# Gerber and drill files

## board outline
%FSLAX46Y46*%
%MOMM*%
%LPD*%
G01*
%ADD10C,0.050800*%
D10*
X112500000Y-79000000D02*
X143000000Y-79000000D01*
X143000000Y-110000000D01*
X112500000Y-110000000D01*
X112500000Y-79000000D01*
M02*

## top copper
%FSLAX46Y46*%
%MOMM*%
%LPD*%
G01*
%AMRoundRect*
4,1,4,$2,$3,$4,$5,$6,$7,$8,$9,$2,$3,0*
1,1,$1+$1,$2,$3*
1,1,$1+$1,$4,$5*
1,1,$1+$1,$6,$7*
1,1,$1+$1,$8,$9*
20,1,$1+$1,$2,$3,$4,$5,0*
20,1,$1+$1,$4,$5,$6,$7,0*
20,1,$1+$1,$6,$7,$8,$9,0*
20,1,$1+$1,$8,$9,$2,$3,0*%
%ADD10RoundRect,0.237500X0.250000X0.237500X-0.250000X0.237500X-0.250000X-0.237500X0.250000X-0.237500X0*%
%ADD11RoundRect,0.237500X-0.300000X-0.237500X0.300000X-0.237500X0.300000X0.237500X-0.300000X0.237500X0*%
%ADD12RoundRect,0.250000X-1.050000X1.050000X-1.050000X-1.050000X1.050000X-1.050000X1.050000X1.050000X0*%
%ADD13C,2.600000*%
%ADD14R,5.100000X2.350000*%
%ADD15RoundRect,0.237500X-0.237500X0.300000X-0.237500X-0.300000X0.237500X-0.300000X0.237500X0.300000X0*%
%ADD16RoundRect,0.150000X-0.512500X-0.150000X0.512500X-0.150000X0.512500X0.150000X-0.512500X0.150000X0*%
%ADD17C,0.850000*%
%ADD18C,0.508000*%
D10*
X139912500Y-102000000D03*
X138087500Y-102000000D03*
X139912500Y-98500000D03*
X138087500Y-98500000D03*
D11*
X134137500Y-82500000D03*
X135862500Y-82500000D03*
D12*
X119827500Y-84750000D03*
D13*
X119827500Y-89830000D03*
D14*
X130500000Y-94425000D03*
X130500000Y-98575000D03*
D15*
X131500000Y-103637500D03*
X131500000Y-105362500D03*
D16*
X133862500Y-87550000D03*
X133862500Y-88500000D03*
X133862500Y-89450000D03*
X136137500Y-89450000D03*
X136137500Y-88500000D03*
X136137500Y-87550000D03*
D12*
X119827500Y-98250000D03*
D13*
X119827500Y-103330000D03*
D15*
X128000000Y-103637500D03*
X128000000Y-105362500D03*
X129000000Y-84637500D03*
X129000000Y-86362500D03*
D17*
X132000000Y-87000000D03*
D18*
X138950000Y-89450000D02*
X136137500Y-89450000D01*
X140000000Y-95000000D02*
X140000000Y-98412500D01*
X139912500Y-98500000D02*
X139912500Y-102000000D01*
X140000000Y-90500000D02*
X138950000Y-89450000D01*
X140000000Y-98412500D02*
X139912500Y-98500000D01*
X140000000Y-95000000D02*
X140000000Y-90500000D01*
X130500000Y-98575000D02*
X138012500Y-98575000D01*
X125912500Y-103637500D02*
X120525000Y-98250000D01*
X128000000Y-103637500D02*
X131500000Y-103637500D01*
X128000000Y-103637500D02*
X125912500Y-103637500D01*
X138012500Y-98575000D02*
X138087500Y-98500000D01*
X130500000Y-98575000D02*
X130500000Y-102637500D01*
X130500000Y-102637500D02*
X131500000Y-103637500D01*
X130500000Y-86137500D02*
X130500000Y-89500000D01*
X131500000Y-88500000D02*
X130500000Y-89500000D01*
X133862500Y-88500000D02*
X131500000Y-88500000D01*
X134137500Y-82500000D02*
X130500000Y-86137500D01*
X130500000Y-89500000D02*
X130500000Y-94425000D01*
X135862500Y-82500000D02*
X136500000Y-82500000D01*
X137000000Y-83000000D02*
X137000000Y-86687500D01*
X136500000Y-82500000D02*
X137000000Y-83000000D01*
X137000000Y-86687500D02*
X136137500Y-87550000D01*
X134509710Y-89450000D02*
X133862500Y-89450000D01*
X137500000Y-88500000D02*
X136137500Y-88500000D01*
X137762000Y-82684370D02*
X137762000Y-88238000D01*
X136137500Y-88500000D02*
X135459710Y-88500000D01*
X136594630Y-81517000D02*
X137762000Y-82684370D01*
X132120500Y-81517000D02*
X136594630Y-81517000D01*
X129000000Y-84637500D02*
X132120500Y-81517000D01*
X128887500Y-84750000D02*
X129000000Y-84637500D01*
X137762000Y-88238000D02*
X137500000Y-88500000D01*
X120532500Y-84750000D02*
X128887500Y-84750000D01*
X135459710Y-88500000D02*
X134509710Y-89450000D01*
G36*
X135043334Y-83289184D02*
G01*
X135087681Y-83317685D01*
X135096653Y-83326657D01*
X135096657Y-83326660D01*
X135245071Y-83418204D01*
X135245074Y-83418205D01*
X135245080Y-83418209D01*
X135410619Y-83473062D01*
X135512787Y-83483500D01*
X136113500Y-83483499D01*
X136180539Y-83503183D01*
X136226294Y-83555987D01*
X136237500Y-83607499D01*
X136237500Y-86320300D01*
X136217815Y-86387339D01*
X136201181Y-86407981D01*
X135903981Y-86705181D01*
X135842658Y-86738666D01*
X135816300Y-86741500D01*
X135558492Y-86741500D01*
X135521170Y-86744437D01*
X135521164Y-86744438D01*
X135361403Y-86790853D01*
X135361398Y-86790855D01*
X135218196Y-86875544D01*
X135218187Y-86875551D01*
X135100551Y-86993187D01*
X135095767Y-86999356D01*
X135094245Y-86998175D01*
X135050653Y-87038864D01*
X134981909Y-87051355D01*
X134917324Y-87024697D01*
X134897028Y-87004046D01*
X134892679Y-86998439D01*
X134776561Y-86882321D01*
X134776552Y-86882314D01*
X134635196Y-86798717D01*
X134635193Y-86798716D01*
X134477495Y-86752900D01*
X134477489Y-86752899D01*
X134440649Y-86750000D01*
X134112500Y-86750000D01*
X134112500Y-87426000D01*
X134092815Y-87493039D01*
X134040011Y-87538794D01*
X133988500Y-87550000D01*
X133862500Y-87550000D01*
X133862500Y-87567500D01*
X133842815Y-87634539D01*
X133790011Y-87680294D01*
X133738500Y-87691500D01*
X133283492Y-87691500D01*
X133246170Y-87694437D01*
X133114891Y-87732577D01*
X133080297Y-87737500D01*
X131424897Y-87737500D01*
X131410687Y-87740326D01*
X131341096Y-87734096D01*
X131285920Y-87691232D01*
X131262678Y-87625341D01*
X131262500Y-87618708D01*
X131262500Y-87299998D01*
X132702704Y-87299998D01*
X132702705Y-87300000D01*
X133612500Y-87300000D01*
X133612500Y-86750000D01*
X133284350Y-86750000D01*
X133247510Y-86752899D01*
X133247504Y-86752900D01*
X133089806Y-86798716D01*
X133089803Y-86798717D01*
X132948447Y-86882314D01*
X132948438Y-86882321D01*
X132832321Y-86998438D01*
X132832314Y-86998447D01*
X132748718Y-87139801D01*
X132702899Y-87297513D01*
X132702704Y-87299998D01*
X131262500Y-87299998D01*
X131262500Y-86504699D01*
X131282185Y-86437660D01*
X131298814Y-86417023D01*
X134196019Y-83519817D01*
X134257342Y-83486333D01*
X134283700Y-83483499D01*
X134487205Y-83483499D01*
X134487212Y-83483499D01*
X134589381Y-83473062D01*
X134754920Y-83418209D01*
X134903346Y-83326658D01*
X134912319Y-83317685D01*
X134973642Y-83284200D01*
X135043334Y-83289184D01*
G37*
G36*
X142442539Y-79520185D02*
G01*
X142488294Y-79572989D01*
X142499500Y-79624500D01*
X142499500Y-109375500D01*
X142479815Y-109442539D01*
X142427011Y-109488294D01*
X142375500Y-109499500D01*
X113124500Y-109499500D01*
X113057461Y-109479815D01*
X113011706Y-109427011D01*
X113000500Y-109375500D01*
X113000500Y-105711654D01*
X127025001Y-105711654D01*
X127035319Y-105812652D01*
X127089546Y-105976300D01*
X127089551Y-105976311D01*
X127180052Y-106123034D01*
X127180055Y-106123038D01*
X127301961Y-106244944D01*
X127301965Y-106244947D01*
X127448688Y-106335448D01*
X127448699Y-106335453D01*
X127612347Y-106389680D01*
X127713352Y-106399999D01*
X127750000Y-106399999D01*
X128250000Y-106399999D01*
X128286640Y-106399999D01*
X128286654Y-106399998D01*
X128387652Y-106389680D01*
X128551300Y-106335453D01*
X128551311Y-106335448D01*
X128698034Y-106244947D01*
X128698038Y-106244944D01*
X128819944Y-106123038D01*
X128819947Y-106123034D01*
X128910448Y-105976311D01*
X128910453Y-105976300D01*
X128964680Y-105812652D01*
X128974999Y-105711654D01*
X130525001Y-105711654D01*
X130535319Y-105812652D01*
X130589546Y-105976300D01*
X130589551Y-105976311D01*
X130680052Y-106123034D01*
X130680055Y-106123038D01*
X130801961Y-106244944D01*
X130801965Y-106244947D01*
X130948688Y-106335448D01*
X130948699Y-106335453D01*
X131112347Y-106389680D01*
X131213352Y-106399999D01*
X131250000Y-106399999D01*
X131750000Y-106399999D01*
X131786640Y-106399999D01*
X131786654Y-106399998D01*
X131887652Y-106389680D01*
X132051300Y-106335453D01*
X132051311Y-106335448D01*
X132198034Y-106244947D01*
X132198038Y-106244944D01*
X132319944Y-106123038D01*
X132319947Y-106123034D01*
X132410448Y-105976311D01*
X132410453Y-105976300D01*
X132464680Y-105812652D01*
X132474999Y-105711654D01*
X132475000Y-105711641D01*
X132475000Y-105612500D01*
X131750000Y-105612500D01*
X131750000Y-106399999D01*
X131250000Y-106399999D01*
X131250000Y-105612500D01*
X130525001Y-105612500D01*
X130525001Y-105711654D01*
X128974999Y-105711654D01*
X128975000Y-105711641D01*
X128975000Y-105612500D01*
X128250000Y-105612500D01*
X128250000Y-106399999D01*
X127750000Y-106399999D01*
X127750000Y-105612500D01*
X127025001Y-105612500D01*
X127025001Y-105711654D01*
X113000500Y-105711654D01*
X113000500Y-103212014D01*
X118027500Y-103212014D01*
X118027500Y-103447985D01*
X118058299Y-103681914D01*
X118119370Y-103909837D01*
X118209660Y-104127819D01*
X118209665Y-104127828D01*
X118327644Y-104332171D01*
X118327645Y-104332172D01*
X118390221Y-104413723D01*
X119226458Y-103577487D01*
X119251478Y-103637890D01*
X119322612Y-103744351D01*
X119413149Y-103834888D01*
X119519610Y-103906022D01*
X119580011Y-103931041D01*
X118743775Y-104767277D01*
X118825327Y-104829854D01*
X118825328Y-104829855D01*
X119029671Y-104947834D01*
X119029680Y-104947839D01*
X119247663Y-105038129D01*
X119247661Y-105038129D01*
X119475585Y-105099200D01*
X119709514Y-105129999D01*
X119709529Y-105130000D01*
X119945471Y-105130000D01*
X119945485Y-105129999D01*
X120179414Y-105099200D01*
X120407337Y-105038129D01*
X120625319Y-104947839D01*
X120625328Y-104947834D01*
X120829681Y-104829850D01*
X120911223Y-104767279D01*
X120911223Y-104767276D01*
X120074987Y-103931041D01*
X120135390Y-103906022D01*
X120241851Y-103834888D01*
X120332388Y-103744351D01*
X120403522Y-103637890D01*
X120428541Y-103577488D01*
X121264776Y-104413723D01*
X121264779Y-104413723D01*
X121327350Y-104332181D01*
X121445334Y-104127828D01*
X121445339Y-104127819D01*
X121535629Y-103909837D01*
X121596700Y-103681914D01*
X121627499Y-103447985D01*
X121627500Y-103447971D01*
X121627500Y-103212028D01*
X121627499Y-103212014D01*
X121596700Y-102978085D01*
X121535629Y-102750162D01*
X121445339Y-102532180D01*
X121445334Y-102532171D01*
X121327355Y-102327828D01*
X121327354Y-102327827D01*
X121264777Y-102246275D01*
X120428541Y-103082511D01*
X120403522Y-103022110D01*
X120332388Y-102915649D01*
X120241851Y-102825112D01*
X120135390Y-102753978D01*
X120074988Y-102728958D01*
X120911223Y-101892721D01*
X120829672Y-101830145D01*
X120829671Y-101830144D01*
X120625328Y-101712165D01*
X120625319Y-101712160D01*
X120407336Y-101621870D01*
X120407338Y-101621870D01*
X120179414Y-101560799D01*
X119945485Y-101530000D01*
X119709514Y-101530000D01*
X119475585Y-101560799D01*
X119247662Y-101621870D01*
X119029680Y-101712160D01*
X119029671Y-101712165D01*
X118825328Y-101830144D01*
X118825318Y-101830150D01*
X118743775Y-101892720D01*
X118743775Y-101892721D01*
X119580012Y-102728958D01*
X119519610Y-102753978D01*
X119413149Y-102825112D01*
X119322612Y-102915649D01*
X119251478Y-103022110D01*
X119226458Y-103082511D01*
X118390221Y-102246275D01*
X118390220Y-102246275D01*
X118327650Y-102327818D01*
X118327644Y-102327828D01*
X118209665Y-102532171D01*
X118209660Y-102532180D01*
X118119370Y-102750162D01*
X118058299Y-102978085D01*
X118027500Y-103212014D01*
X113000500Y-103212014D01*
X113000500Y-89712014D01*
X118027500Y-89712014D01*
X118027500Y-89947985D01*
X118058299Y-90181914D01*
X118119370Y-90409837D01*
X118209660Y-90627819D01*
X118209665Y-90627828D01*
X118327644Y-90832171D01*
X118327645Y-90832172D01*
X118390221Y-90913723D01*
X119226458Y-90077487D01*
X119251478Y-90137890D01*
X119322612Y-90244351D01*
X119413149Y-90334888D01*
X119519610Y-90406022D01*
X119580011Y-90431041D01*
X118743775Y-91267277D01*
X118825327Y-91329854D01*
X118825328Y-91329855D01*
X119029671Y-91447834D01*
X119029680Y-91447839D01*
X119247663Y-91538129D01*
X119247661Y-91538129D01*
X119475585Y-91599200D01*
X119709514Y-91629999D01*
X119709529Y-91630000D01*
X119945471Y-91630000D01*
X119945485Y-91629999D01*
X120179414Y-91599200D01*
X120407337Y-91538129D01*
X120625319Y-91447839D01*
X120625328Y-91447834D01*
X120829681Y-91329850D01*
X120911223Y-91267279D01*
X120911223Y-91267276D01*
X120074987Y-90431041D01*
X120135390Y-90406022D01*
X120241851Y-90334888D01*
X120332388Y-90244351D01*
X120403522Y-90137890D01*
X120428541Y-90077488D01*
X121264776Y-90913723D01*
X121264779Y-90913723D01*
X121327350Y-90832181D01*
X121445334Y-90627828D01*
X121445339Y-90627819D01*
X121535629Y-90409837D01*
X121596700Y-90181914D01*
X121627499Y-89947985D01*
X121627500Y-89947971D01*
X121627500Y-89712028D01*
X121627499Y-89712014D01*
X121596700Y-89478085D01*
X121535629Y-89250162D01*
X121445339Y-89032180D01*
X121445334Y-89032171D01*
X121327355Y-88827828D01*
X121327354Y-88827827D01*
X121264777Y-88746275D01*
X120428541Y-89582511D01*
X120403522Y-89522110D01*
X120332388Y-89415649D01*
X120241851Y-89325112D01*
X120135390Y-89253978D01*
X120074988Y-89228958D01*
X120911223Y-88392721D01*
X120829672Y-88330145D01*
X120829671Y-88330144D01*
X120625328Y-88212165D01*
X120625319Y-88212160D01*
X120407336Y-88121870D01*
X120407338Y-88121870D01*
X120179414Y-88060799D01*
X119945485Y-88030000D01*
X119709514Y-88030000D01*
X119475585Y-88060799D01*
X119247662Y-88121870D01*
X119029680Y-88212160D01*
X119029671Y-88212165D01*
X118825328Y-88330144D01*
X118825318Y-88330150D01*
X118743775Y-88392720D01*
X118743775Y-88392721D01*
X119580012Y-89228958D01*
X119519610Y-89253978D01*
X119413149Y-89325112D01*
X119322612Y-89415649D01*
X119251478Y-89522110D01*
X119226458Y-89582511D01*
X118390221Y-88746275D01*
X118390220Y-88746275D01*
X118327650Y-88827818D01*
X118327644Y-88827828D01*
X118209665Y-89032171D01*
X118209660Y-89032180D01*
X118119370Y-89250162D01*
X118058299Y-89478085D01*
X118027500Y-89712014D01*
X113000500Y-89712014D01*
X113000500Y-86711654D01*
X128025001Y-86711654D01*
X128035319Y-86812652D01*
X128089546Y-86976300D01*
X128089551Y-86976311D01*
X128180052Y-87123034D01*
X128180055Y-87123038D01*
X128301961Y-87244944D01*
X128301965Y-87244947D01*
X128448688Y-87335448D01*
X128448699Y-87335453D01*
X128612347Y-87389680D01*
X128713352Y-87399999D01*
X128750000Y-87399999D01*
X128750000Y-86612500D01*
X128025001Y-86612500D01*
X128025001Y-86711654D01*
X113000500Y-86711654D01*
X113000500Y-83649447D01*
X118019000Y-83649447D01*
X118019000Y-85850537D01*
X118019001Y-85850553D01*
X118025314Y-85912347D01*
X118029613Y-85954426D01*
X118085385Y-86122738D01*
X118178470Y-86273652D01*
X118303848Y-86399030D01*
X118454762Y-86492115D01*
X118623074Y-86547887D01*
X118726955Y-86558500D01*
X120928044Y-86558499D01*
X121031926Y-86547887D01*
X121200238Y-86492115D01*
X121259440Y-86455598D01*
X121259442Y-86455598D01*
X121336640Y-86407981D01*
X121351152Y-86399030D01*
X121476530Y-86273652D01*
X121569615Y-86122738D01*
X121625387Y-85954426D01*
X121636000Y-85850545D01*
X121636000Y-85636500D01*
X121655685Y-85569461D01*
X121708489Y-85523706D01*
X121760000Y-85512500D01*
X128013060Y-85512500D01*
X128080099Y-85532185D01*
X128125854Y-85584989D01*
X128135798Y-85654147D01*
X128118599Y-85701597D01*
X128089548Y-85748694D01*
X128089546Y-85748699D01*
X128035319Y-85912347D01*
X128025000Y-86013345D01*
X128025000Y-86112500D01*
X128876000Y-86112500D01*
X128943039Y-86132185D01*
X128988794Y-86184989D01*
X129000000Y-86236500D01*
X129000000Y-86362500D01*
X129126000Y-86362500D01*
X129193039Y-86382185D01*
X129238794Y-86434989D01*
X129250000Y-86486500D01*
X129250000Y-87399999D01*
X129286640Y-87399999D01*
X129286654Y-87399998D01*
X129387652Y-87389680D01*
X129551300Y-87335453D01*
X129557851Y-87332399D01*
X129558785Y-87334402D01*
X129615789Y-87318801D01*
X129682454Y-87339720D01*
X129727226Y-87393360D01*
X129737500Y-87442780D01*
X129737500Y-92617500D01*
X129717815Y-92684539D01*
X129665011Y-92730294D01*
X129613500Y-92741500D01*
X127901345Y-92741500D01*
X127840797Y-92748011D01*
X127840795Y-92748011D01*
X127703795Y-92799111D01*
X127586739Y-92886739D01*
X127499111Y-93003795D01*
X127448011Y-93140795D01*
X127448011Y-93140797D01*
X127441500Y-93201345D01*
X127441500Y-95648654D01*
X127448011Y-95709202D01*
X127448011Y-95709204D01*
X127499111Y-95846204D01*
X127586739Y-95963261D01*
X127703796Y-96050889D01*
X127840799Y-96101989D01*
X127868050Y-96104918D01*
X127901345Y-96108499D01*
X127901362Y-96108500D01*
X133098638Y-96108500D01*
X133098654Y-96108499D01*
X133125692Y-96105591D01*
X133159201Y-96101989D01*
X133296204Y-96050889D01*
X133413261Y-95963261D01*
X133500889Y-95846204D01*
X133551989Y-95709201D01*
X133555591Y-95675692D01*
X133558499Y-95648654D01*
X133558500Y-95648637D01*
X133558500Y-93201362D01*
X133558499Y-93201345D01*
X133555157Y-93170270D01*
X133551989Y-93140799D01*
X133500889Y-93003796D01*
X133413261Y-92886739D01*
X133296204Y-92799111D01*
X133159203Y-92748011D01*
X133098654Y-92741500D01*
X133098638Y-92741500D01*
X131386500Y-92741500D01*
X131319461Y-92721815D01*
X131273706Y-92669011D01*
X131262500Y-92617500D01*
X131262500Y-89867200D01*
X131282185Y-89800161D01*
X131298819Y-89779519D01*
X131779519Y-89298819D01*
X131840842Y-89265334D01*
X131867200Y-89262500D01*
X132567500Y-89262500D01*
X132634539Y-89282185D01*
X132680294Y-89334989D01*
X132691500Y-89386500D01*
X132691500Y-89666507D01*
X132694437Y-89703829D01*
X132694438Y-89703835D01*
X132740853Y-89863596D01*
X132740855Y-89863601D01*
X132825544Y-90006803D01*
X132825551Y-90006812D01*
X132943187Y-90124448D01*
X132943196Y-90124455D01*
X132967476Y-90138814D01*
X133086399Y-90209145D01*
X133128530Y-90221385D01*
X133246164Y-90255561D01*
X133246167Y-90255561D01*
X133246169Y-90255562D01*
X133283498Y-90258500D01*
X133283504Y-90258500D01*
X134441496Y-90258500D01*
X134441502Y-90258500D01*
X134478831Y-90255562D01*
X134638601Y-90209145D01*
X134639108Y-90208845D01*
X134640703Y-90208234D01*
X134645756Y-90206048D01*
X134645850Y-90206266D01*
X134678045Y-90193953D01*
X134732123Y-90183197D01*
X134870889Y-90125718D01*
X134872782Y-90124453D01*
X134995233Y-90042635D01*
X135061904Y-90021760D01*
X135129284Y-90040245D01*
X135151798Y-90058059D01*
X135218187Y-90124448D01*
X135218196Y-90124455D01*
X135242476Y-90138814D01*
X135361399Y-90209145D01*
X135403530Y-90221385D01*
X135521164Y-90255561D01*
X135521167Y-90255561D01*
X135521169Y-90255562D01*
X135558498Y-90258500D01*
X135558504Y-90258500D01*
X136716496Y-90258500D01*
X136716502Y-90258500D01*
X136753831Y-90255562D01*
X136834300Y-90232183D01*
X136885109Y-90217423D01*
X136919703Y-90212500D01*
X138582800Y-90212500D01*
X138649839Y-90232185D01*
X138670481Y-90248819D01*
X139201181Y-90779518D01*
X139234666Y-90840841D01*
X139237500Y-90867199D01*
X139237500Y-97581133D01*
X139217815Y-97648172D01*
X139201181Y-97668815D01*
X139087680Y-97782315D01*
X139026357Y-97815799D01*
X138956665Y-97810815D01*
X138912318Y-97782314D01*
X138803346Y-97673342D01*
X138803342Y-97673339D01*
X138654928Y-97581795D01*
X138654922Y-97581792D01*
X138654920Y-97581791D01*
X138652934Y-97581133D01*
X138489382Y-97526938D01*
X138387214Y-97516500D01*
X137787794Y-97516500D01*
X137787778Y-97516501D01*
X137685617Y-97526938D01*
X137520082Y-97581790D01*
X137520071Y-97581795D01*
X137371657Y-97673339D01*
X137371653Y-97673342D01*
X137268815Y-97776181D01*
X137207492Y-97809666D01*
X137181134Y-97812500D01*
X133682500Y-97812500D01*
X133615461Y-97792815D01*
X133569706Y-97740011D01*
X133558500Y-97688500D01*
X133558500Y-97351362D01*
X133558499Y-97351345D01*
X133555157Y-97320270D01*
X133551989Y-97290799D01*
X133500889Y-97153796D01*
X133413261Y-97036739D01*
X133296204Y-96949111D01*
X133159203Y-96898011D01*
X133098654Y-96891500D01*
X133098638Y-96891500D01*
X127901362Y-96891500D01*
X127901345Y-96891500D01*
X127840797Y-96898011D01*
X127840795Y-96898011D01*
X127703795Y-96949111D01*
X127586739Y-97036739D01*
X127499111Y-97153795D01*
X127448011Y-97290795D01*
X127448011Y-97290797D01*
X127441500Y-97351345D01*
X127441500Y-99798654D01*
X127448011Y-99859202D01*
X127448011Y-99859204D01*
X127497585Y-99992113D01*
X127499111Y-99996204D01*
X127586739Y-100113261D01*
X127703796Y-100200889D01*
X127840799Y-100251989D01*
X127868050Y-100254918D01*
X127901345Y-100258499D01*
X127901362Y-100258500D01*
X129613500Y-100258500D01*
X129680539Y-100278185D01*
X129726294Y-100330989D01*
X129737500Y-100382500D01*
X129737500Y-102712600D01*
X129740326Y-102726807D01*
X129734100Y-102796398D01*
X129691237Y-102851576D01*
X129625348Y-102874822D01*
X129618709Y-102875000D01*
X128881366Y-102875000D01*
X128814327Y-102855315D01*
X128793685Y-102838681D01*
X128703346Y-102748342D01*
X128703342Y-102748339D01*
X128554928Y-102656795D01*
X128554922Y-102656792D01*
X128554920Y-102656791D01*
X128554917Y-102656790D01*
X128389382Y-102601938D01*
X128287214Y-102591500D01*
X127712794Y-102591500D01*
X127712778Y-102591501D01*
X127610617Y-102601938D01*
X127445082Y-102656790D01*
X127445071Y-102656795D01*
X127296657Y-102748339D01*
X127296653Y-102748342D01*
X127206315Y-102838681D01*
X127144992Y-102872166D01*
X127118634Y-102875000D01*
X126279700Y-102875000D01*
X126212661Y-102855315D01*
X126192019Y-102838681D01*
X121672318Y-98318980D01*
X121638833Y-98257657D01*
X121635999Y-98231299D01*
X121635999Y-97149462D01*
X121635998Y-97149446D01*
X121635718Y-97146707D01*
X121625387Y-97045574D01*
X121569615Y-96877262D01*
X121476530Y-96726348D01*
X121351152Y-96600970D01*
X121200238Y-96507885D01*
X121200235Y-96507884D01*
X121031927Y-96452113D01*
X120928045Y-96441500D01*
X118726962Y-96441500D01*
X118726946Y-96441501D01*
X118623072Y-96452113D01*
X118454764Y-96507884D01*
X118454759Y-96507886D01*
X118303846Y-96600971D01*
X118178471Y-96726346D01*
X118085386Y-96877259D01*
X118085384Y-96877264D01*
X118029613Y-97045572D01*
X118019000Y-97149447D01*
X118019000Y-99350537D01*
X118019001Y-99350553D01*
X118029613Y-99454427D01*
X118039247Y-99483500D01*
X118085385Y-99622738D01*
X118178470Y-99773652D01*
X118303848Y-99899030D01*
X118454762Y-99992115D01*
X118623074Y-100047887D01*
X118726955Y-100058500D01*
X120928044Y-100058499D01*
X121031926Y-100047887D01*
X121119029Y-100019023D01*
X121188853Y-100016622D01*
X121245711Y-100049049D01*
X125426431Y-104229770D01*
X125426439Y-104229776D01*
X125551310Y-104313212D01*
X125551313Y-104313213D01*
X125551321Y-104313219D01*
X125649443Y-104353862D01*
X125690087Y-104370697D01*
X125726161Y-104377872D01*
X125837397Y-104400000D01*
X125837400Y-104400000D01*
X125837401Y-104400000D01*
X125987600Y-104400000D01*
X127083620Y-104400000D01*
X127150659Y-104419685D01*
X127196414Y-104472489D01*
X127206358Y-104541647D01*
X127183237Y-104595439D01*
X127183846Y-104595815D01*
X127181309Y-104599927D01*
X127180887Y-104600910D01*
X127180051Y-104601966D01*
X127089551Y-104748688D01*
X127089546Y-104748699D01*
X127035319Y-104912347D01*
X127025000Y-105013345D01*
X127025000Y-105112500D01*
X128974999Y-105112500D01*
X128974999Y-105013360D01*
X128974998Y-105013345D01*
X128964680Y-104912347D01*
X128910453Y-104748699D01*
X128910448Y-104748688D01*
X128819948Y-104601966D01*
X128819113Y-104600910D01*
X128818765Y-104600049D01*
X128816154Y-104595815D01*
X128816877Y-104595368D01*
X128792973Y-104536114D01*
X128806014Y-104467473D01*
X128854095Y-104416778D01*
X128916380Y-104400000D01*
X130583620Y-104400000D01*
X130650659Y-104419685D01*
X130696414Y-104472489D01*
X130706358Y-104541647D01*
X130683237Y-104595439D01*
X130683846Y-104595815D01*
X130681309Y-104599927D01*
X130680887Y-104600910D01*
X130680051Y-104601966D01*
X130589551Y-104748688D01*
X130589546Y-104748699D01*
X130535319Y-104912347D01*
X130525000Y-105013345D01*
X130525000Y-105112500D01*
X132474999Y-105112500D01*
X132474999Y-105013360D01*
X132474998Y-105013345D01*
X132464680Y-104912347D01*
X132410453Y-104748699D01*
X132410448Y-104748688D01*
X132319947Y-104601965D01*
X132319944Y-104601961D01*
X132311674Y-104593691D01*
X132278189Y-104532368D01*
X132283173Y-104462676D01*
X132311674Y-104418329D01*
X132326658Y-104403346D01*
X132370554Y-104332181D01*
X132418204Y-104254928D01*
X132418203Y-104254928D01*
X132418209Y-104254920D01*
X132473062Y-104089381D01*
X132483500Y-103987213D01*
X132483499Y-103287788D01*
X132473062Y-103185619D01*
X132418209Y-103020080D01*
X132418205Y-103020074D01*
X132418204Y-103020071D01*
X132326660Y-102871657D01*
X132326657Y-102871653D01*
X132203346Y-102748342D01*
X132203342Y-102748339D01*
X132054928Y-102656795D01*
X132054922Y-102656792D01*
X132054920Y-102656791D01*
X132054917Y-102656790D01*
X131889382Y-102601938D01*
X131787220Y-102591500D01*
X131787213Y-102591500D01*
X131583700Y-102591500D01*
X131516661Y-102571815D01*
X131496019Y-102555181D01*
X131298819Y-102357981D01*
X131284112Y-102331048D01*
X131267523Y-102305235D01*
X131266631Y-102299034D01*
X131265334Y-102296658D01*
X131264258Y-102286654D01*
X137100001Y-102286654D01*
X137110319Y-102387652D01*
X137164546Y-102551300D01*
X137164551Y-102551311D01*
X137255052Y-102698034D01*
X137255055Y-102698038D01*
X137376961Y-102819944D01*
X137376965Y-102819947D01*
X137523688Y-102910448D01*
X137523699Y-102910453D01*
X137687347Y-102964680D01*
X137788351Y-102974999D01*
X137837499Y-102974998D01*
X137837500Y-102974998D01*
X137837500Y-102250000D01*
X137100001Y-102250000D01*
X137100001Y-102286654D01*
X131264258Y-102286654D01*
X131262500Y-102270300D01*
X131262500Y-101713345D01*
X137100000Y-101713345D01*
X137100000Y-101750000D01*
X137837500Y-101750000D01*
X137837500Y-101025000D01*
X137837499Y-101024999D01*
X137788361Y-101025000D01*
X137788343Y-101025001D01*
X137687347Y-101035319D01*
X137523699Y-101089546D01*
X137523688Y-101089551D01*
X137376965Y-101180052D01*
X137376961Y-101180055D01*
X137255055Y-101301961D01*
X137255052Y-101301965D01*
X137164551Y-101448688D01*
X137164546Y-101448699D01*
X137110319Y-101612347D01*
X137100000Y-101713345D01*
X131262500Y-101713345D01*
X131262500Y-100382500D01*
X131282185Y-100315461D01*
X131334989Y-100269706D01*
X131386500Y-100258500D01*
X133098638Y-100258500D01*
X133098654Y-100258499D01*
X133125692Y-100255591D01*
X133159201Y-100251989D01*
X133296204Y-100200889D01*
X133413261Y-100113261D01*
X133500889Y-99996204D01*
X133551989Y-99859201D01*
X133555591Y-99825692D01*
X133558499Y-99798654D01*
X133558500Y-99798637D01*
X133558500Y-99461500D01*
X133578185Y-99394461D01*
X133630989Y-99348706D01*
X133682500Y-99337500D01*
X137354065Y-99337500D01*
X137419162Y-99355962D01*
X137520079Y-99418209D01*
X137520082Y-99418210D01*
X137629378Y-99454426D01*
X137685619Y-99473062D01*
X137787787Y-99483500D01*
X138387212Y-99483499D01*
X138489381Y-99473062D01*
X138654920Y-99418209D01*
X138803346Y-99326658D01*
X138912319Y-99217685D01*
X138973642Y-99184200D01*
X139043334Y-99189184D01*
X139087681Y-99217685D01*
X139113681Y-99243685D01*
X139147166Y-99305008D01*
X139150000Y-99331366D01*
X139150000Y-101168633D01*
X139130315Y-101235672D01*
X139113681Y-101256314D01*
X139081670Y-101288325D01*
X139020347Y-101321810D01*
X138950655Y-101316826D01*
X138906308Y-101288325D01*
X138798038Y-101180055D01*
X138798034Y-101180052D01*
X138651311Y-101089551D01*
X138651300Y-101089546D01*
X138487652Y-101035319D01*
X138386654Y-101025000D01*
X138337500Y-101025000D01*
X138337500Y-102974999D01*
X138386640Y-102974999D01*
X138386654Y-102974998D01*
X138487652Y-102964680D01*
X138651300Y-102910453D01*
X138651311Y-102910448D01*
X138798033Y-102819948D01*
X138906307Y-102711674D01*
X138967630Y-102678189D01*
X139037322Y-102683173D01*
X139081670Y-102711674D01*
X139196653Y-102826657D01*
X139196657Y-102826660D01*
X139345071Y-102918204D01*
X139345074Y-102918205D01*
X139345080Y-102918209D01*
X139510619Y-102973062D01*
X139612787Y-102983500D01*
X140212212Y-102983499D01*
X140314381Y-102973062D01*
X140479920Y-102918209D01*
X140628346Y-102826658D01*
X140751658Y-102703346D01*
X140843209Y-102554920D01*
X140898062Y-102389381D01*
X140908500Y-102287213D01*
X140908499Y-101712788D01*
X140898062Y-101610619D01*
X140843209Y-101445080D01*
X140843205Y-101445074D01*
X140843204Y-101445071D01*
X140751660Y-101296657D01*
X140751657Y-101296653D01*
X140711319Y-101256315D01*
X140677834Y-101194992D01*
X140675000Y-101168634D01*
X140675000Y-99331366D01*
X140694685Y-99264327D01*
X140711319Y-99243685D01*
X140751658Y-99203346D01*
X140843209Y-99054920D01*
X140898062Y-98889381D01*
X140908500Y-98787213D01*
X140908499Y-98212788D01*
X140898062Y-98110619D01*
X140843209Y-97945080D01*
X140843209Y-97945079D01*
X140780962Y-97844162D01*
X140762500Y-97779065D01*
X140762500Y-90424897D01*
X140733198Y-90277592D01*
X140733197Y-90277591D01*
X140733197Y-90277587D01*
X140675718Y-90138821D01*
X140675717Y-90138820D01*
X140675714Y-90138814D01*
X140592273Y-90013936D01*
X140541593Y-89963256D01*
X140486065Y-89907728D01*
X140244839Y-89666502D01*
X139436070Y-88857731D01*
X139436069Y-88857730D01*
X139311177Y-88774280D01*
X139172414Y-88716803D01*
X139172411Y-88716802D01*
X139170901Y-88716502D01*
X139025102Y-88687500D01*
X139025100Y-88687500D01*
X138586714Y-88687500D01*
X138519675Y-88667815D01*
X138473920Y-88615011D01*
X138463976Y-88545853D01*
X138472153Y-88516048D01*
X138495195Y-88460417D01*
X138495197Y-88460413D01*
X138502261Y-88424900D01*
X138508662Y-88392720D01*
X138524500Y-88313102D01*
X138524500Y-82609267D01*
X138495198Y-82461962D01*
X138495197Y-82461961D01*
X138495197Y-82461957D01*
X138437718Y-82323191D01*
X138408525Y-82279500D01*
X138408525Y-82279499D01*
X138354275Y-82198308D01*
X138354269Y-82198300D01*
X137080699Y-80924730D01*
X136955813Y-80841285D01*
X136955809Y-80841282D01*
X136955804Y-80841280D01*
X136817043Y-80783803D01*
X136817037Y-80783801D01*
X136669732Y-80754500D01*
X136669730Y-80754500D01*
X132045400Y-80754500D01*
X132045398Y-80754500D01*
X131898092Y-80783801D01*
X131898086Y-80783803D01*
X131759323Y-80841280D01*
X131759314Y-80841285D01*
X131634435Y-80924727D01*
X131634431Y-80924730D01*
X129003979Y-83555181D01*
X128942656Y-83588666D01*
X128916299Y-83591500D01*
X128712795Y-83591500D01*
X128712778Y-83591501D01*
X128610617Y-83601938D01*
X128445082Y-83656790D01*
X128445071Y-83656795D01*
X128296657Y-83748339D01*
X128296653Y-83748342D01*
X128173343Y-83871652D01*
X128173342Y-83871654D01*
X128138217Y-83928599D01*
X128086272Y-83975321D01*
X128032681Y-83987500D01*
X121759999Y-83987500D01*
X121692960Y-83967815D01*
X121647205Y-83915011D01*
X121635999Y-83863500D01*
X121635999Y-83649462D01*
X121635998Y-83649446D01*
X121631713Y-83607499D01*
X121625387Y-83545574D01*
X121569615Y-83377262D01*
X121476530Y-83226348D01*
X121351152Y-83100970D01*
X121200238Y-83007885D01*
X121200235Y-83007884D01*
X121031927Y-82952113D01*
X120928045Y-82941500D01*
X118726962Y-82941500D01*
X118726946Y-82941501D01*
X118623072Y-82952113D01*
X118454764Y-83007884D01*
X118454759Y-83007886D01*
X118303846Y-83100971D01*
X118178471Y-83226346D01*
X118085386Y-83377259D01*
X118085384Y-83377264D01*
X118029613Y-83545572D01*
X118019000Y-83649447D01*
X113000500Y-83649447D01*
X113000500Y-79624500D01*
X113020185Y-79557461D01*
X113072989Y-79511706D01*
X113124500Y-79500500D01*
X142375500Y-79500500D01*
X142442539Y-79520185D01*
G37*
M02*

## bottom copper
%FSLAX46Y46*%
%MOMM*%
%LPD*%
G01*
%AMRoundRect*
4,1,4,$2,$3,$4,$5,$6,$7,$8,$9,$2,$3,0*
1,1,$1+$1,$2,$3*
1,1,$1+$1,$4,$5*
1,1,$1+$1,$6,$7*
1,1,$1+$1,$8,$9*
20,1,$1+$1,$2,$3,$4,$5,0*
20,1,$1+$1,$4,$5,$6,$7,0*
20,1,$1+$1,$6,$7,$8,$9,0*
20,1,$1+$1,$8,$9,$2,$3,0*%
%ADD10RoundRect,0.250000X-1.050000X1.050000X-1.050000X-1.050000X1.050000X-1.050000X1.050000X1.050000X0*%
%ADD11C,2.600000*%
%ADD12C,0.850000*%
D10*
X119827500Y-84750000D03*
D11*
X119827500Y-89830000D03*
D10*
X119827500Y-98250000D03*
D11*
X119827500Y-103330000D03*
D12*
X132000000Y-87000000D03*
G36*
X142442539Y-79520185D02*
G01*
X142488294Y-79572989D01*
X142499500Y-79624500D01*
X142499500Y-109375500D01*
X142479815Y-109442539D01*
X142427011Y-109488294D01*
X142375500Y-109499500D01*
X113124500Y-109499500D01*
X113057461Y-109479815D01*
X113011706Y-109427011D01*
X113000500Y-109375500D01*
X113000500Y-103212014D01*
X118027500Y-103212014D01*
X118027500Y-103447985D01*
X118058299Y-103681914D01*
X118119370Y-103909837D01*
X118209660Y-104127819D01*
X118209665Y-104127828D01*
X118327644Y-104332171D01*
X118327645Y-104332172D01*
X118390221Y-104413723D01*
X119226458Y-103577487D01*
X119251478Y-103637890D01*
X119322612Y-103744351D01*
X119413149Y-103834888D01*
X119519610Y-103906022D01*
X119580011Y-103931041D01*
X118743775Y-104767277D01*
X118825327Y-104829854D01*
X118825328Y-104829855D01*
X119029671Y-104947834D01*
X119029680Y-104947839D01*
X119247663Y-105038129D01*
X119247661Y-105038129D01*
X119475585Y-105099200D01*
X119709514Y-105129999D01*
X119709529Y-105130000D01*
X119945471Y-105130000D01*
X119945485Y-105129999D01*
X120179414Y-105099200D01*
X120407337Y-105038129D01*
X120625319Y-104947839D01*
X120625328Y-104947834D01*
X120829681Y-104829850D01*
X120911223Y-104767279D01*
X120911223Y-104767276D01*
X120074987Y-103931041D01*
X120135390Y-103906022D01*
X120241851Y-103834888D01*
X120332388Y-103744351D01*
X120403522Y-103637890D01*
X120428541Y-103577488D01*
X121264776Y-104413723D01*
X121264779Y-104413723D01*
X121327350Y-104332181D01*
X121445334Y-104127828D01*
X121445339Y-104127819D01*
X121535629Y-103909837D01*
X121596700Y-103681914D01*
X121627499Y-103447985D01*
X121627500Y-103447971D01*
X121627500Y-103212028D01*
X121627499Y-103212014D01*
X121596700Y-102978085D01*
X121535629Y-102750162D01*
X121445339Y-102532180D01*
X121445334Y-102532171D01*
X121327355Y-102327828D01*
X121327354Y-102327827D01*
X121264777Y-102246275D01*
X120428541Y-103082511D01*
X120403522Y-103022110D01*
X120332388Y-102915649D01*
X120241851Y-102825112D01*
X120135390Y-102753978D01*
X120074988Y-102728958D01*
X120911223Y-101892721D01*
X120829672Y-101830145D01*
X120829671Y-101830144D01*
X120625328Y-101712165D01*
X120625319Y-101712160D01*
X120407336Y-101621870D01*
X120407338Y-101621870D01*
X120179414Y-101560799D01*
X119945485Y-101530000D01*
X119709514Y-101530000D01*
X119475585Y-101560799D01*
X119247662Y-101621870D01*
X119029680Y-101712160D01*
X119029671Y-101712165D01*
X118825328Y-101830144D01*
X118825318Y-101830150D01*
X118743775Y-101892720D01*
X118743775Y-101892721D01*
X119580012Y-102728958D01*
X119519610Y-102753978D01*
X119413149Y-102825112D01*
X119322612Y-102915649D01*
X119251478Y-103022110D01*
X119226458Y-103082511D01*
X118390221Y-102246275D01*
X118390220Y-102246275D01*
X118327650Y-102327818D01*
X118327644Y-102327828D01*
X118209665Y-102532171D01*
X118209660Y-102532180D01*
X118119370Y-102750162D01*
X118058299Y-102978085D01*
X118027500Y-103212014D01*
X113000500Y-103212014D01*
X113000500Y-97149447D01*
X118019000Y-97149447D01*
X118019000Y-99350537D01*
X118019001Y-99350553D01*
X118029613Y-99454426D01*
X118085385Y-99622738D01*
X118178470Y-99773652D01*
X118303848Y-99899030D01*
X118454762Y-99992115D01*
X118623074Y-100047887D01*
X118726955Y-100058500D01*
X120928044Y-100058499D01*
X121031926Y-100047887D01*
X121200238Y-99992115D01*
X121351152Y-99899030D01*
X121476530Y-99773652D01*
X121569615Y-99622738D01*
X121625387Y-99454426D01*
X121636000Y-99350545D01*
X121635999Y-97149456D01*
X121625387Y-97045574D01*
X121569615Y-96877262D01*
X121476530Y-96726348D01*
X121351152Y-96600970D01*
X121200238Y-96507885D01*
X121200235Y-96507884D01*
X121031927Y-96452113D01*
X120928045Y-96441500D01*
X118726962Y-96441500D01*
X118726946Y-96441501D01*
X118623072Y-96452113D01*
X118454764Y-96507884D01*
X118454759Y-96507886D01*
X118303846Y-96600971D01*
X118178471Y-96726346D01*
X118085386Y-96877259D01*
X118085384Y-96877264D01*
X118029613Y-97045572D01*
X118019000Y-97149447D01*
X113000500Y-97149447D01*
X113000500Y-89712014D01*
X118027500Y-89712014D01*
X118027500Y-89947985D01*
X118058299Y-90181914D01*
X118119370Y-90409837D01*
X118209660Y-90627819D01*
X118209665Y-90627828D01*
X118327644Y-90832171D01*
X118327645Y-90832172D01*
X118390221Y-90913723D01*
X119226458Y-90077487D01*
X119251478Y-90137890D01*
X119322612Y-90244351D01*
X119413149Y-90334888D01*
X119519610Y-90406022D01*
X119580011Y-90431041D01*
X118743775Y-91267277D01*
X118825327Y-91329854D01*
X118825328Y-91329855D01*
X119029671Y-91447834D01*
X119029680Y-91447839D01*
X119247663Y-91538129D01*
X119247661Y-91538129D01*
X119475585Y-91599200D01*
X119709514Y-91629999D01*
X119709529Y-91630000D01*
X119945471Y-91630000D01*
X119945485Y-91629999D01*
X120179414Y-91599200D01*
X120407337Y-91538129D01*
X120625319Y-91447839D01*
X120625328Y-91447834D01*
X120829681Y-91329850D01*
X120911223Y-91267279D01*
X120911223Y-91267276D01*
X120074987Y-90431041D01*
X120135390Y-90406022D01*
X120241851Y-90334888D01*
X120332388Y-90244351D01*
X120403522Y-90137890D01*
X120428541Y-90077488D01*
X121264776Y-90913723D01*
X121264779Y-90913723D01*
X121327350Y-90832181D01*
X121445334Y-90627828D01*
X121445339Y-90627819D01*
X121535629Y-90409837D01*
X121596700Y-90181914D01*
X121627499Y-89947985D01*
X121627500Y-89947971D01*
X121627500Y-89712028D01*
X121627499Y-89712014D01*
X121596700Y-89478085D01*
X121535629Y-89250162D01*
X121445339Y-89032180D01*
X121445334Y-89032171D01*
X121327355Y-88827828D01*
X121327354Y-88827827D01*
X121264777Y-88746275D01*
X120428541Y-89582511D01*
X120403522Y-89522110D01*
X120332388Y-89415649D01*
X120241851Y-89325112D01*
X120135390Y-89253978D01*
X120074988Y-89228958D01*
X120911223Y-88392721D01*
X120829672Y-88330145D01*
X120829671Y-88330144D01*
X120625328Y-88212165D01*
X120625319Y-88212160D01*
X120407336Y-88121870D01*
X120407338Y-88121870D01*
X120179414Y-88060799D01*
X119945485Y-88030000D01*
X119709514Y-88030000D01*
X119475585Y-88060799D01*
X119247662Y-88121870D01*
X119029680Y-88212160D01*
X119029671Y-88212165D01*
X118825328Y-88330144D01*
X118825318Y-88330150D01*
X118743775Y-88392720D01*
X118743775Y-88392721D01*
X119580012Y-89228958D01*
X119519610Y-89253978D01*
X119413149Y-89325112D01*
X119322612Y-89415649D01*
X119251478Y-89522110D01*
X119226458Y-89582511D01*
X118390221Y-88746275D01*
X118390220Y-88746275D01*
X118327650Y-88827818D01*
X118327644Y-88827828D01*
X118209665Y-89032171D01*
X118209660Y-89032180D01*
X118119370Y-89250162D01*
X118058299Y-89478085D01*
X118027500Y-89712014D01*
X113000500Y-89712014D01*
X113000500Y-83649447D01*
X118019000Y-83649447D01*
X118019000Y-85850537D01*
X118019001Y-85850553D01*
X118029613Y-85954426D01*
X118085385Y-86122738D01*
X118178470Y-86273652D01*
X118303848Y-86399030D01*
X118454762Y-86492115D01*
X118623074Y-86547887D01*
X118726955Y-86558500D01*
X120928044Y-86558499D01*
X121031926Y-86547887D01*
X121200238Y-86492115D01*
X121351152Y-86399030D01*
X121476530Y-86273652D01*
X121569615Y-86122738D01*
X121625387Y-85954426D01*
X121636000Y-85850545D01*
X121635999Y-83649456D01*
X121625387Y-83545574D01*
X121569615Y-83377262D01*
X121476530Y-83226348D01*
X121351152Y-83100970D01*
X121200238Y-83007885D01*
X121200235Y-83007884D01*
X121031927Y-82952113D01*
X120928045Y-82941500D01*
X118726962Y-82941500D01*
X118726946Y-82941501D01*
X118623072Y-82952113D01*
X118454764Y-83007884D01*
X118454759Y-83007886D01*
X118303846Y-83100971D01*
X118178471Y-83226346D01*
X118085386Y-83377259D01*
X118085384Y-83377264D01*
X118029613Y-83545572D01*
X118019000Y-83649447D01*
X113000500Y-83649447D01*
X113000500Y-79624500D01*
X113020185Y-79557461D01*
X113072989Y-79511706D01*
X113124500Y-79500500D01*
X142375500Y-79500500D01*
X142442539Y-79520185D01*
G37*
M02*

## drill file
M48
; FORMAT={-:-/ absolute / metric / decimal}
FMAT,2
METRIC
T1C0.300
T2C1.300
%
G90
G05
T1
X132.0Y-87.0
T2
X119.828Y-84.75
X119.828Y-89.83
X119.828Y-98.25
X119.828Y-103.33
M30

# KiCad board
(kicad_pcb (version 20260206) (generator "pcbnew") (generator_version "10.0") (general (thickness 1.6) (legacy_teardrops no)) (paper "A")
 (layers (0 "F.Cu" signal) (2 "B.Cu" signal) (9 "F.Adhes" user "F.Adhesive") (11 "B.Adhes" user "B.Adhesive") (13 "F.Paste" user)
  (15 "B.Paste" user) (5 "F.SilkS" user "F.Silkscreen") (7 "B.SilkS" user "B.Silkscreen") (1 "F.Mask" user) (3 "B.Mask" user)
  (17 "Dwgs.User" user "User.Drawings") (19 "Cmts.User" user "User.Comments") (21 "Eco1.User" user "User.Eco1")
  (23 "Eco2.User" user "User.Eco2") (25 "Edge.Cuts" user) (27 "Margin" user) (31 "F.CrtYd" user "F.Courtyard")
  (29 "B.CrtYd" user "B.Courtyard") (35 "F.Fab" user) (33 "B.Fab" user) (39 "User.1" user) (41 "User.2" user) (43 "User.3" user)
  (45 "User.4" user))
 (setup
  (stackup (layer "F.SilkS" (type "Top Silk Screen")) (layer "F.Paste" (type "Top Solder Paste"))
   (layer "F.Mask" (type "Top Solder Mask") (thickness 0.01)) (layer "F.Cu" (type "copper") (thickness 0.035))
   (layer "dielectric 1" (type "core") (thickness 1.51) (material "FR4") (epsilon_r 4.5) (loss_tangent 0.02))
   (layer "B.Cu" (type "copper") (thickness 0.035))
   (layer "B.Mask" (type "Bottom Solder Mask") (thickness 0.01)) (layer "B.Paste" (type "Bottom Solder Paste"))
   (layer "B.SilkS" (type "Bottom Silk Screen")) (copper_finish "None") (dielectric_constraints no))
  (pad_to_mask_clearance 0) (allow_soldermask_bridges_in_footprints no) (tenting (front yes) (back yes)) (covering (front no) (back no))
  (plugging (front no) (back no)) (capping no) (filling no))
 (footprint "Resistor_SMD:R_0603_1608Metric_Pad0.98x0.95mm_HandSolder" (layer "F.Cu") (at 139 102 180)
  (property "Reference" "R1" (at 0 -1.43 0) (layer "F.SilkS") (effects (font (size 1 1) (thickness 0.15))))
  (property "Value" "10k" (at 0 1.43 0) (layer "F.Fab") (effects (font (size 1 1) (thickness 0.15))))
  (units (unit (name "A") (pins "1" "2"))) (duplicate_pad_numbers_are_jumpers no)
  (pad "1" smd roundrect (at -0.9125 0 180) (size 0.975 0.95) (layers "F.Cu" "F.Mask" "F.Paste") (roundrect_rratio 0.25)
   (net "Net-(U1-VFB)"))
  (pad "2" smd roundrect (at 0.9125 0 180) (size 0.975 0.95) (layers "F.Cu" "F.Mask" "F.Paste") (roundrect_rratio 0.25) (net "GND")))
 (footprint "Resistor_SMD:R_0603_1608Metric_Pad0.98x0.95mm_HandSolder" (layer "F.Cu") (at 139 98.5 180)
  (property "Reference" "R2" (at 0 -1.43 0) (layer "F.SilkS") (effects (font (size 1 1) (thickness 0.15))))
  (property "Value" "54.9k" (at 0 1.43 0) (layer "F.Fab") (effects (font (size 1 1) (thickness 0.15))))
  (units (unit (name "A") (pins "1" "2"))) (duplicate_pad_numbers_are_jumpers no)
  (pad "1" smd roundrect (at -0.9125 0 180) (size 0.975 0.95) (layers "F.Cu" "F.Mask" "F.Paste") (roundrect_rratio 0.25)
   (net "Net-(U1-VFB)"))
  (pad "2" smd roundrect (at 0.9125 0 180) (size 0.975 0.95) (layers "F.Cu" "F.Mask" "F.Paste") (roundrect_rratio 0.25) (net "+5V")))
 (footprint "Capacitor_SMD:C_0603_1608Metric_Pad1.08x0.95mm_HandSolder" (layer "F.Cu") (at 135 82.5)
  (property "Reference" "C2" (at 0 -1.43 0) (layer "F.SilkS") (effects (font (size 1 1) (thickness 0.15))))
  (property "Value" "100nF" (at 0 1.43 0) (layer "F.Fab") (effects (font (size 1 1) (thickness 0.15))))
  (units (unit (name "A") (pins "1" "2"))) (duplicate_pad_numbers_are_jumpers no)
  (pad "1" smd roundrect (at -0.8625 0) (size 1.075 0.95) (layers "F.Cu" "F.Mask" "F.Paste") (roundrect_rratio 0.25) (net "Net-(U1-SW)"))
  (pad "2" smd roundrect (at 0.8625 0) (size 1.075 0.95) (layers "F.Cu" "F.Mask" "F.Paste") (roundrect_rratio 0.25) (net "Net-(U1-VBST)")))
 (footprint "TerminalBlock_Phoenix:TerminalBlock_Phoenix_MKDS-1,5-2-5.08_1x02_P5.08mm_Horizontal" (layer "F.Cu") (at 119.8275 84.75 -90)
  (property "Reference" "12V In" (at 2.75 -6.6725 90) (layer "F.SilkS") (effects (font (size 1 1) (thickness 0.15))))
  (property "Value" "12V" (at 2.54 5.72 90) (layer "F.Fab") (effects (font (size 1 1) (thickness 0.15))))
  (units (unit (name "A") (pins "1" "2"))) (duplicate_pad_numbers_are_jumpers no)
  (pad "1" thru_hole roundrect (at 0 0 270) (size 2.6 2.6) (drill 1.3) (layers "*.Cu" "*.Mask") (remove_unused_layers no)
   (roundrect_rratio 0.096154) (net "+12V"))
  (pad "2" thru_hole circle (at 5.08 0 270) (size 2.6 2.6) (drill 1.3) (layers "*.Cu" "*.Mask") (remove_unused_layers no) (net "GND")))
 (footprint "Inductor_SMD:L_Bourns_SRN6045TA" (layer "F.Cu") (at 130.5 96.5 -90)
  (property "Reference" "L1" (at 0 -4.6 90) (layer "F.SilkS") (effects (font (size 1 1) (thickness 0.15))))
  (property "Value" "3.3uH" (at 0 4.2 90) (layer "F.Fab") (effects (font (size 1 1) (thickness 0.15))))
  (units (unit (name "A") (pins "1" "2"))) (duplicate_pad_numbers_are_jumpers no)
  (pad "1" smd rect (at -2.075 0 270) (size 2.35 5.1) (layers "F.Cu" "F.Mask" "F.Paste") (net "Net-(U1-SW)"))
  (pad "2" smd rect (at 2.075 0 270) (size 2.35 5.1) (layers "F.Cu" "F.Mask" "F.Paste") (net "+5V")))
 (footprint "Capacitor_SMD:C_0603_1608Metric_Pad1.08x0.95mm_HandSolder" (layer "F.Cu") (at 131.5 104.5 -90)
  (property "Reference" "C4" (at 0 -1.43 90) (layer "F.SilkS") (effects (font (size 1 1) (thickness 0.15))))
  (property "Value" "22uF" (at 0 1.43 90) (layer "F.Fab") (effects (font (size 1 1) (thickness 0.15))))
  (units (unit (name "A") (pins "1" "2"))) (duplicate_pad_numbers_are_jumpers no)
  (pad "1" smd roundrect (at -0.8625 0 270) (size 1.075 0.95) (layers "F.Cu" "F.Mask" "F.Paste") (roundrect_rratio 0.25) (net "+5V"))
  (pad "2" smd roundrect (at 0.8625 0 270) (size 1.075 0.95) (layers "F.Cu" "F.Mask" "F.Paste") (roundrect_rratio 0.25) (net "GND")))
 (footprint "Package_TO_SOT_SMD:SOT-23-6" (layer "F.Cu") (at 135 88.5)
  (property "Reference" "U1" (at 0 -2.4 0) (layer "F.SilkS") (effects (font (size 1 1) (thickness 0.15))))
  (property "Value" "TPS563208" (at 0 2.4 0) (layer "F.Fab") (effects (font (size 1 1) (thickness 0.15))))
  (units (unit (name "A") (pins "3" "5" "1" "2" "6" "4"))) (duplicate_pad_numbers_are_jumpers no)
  (pad "1" smd roundrect (at -1.1375 -0.95) (size 1.325 0.6) (layers "F.Cu" "F.Mask" "F.Paste") (roundrect_rratio 0.25) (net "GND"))
  (pad "2" smd roundrect (at -1.1375 0) (size 1.325 0.6) (layers "F.Cu" "F.Mask" "F.Paste") (roundrect_rratio 0.25) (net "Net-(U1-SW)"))
  (pad "3" smd roundrect (at -1.1375 0.95) (size 1.325 0.6) (layers "F.Cu" "F.Mask" "F.Paste") (roundrect_rratio 0.25) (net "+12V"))
  (pad "4" smd roundrect (at 1.1375 0.95) (size 1.325 0.6) (layers "F.Cu" "F.Mask" "F.Paste") (roundrect_rratio 0.25) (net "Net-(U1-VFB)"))
  (pad "5" smd roundrect (at 1.1375 0) (size 1.325 0.6) (layers "F.Cu" "F.Mask" "F.Paste") (roundrect_rratio 0.25) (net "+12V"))
  (pad "6" smd roundrect (at 1.1375 -0.95) (size 1.325 0.6) (layers "F.Cu" "F.Mask" "F.Paste") (roundrect_rratio 0.25) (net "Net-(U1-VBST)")))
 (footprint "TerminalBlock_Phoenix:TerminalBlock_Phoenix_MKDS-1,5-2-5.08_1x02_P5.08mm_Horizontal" (layer "F.Cu") (at 119.8275 98.25 -90)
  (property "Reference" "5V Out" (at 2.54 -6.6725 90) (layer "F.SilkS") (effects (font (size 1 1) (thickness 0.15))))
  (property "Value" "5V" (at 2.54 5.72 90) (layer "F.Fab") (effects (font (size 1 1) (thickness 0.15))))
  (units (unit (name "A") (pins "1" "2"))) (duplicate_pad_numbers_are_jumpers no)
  (pad "1" thru_hole roundrect (at 0 0 270) (size 2.6 2.6) (drill 1.3) (layers "*.Cu" "*.Mask") (remove_unused_layers no)
   (roundrect_rratio 0.096154) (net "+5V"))
  (pad "2" thru_hole circle (at 5.08 0 270) (size 2.6 2.6) (drill 1.3) (layers "*.Cu" "*.Mask") (remove_unused_layers no) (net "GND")))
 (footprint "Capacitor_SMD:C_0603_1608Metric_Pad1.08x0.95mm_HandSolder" (layer "F.Cu") (at 128 104.5 -90)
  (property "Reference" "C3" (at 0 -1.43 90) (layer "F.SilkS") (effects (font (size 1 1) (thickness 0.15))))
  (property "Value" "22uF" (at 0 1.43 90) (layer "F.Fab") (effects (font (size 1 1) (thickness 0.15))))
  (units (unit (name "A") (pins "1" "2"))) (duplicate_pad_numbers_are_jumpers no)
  (pad "1" smd roundrect (at -0.8625 0 270) (size 1.075 0.95) (layers "F.Cu" "F.Mask" "F.Paste") (roundrect_rratio 0.25) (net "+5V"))
  (pad "2" smd roundrect (at 0.8625 0 270) (size 1.075 0.95) (layers "F.Cu" "F.Mask" "F.Paste") (roundrect_rratio 0.25) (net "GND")))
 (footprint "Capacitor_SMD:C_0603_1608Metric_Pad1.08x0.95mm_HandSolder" (layer "F.Cu") (at 129 85.5 -90)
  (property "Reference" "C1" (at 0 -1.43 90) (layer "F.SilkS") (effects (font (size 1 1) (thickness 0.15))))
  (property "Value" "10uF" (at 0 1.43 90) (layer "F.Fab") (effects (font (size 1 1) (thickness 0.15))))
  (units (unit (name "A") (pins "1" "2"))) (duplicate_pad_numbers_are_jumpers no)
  (pad "1" smd roundrect (at -0.8625 0 270) (size 1.075 0.95) (layers "F.Cu" "F.Mask" "F.Paste") (roundrect_rratio 0.25) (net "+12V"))
  (pad "2" smd roundrect (at 0.8625 0 270) (size 1.075 0.95) (layers "F.Cu" "F.Mask" "F.Paste") (roundrect_rratio 0.25) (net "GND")))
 (gr_rect (start 112.5 79) (end 143 110) (stroke (width 0.0508) (type default)) (fill no) (layer "Edge.Cuts"))
 (segment (start 138.95 89.45) (end 136.1375 89.45) (width 0.508) (layer "F.Cu") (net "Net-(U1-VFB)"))
 (segment (start 140 95) (end 140 98.4125) (width 0.508) (layer "F.Cu") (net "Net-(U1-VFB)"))
 (segment (start 139.9125 98.5) (end 139.9125 102) (width 0.508) (layer "F.Cu") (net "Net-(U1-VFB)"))
 (segment (start 140 90.5) (end 138.95 89.45) (width 0.508) (layer "F.Cu") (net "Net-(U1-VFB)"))
 (segment (start 140 98.4125) (end 139.9125 98.5) (width 0.508) (layer "F.Cu") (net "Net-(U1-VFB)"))
 (segment (start 140 95) (end 140 90.5) (width 0.508) (layer "F.Cu") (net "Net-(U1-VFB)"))
 (via (at 132 87) (size 0.85) (drill 0.3) (layers "F.Cu" "B.Cu") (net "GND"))
 (segment (start 130.5 98.575) (end 138.0125 98.575) (width 0.508) (layer "F.Cu") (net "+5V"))
 (segment (start 125.9125 103.6375) (end 120.525 98.25) (width 0.508) (layer "F.Cu") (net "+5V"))
 (segment (start 128 103.6375) (end 131.5 103.6375) (width 0.508) (layer "F.Cu") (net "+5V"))
 (segment (start 128 103.6375) (end 125.9125 103.6375) (width 0.508) (layer "F.Cu") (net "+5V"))
 (segment (start 138.0125 98.575) (end 138.0875 98.5) (width 0.508) (layer "F.Cu") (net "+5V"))
 (segment (start 130.5 98.575) (end 130.5 102.6375) (width 0.508) (layer "F.Cu") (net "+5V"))
 (segment (start 130.5 102.6375) (end 131.5 103.6375) (width 0.508) (layer "F.Cu") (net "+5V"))
 (segment (start 130.5 86.1375) (end 130.5 89.5) (width 0.508) (layer "F.Cu") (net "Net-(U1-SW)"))
 (segment (start 131.5 88.5) (end 130.5 89.5) (width 0.508) (layer "F.Cu") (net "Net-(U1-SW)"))
 (segment (start 133.8625 88.5) (end 131.5 88.5) (width 0.508) (layer "F.Cu") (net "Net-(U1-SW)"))
 (segment (start 134.1375 82.5) (end 130.5 86.1375) (width 0.508) (layer "F.Cu") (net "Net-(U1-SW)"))
 (segment (start 130.5 89.5) (end 130.5 94.425) (width 0.508) (layer "F.Cu") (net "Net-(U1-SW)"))
 (segment (start 135.8625 82.5) (end 136.5 82.5) (width 0.508) (layer "F.Cu") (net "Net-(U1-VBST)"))
 (segment (start 137 83) (end 137 86.6875) (width 0.508) (layer "F.Cu") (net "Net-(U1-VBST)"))
 (segment (start 136.5 82.5) (end 137 83) (width 0.508) (layer "F.Cu") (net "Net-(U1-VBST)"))
 (segment (start 137 86.6875) (end 136.1375 87.55) (width 0.508) (layer "F.Cu") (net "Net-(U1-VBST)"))
 (segment (start 134.50971 89.45) (end 133.8625 89.45) (width 0.508) (layer "F.Cu") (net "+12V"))
 (segment (start 137.5 88.5) (end 136.1375 88.5) (width 0.508) (layer "F.Cu") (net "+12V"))
 (segment (start 137.762 82.68437) (end 137.762 88.238) (width 0.508) (layer "F.Cu") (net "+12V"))
 (segment (start 136.1375 88.5) (end 135.45971 88.5) (width 0.508) (layer "F.Cu") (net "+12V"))
 (segment (start 136.59463 81.517) (end 137.762 82.68437) (width 0.508) (layer "F.Cu") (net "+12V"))
 (segment (start 132.1205 81.517) (end 136.59463 81.517) (width 0.508) (layer "F.Cu") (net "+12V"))
 (segment (start 129 84.6375) (end 132.1205 81.517) (width 0.508) (layer "F.Cu") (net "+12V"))
 (segment (start 128.8875 84.75) (end 129 84.6375) (width 0.508) (layer "F.Cu") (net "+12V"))
 (segment (start 137.762 88.238) (end 137.5 88.5) (width 0.508) (layer "F.Cu") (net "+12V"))
 (segment (start 120.5325 84.75) (end 128.8875 84.75) (width 0.508) (layer "F.Cu") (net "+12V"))
 (segment (start 135.45971 88.5) (end 134.50971 89.45) (width 0.508) (layer "F.Cu") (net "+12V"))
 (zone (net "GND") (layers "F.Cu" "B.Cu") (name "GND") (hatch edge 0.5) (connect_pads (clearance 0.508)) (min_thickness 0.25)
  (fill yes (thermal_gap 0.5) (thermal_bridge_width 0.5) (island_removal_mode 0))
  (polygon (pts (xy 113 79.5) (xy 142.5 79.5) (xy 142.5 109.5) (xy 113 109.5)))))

